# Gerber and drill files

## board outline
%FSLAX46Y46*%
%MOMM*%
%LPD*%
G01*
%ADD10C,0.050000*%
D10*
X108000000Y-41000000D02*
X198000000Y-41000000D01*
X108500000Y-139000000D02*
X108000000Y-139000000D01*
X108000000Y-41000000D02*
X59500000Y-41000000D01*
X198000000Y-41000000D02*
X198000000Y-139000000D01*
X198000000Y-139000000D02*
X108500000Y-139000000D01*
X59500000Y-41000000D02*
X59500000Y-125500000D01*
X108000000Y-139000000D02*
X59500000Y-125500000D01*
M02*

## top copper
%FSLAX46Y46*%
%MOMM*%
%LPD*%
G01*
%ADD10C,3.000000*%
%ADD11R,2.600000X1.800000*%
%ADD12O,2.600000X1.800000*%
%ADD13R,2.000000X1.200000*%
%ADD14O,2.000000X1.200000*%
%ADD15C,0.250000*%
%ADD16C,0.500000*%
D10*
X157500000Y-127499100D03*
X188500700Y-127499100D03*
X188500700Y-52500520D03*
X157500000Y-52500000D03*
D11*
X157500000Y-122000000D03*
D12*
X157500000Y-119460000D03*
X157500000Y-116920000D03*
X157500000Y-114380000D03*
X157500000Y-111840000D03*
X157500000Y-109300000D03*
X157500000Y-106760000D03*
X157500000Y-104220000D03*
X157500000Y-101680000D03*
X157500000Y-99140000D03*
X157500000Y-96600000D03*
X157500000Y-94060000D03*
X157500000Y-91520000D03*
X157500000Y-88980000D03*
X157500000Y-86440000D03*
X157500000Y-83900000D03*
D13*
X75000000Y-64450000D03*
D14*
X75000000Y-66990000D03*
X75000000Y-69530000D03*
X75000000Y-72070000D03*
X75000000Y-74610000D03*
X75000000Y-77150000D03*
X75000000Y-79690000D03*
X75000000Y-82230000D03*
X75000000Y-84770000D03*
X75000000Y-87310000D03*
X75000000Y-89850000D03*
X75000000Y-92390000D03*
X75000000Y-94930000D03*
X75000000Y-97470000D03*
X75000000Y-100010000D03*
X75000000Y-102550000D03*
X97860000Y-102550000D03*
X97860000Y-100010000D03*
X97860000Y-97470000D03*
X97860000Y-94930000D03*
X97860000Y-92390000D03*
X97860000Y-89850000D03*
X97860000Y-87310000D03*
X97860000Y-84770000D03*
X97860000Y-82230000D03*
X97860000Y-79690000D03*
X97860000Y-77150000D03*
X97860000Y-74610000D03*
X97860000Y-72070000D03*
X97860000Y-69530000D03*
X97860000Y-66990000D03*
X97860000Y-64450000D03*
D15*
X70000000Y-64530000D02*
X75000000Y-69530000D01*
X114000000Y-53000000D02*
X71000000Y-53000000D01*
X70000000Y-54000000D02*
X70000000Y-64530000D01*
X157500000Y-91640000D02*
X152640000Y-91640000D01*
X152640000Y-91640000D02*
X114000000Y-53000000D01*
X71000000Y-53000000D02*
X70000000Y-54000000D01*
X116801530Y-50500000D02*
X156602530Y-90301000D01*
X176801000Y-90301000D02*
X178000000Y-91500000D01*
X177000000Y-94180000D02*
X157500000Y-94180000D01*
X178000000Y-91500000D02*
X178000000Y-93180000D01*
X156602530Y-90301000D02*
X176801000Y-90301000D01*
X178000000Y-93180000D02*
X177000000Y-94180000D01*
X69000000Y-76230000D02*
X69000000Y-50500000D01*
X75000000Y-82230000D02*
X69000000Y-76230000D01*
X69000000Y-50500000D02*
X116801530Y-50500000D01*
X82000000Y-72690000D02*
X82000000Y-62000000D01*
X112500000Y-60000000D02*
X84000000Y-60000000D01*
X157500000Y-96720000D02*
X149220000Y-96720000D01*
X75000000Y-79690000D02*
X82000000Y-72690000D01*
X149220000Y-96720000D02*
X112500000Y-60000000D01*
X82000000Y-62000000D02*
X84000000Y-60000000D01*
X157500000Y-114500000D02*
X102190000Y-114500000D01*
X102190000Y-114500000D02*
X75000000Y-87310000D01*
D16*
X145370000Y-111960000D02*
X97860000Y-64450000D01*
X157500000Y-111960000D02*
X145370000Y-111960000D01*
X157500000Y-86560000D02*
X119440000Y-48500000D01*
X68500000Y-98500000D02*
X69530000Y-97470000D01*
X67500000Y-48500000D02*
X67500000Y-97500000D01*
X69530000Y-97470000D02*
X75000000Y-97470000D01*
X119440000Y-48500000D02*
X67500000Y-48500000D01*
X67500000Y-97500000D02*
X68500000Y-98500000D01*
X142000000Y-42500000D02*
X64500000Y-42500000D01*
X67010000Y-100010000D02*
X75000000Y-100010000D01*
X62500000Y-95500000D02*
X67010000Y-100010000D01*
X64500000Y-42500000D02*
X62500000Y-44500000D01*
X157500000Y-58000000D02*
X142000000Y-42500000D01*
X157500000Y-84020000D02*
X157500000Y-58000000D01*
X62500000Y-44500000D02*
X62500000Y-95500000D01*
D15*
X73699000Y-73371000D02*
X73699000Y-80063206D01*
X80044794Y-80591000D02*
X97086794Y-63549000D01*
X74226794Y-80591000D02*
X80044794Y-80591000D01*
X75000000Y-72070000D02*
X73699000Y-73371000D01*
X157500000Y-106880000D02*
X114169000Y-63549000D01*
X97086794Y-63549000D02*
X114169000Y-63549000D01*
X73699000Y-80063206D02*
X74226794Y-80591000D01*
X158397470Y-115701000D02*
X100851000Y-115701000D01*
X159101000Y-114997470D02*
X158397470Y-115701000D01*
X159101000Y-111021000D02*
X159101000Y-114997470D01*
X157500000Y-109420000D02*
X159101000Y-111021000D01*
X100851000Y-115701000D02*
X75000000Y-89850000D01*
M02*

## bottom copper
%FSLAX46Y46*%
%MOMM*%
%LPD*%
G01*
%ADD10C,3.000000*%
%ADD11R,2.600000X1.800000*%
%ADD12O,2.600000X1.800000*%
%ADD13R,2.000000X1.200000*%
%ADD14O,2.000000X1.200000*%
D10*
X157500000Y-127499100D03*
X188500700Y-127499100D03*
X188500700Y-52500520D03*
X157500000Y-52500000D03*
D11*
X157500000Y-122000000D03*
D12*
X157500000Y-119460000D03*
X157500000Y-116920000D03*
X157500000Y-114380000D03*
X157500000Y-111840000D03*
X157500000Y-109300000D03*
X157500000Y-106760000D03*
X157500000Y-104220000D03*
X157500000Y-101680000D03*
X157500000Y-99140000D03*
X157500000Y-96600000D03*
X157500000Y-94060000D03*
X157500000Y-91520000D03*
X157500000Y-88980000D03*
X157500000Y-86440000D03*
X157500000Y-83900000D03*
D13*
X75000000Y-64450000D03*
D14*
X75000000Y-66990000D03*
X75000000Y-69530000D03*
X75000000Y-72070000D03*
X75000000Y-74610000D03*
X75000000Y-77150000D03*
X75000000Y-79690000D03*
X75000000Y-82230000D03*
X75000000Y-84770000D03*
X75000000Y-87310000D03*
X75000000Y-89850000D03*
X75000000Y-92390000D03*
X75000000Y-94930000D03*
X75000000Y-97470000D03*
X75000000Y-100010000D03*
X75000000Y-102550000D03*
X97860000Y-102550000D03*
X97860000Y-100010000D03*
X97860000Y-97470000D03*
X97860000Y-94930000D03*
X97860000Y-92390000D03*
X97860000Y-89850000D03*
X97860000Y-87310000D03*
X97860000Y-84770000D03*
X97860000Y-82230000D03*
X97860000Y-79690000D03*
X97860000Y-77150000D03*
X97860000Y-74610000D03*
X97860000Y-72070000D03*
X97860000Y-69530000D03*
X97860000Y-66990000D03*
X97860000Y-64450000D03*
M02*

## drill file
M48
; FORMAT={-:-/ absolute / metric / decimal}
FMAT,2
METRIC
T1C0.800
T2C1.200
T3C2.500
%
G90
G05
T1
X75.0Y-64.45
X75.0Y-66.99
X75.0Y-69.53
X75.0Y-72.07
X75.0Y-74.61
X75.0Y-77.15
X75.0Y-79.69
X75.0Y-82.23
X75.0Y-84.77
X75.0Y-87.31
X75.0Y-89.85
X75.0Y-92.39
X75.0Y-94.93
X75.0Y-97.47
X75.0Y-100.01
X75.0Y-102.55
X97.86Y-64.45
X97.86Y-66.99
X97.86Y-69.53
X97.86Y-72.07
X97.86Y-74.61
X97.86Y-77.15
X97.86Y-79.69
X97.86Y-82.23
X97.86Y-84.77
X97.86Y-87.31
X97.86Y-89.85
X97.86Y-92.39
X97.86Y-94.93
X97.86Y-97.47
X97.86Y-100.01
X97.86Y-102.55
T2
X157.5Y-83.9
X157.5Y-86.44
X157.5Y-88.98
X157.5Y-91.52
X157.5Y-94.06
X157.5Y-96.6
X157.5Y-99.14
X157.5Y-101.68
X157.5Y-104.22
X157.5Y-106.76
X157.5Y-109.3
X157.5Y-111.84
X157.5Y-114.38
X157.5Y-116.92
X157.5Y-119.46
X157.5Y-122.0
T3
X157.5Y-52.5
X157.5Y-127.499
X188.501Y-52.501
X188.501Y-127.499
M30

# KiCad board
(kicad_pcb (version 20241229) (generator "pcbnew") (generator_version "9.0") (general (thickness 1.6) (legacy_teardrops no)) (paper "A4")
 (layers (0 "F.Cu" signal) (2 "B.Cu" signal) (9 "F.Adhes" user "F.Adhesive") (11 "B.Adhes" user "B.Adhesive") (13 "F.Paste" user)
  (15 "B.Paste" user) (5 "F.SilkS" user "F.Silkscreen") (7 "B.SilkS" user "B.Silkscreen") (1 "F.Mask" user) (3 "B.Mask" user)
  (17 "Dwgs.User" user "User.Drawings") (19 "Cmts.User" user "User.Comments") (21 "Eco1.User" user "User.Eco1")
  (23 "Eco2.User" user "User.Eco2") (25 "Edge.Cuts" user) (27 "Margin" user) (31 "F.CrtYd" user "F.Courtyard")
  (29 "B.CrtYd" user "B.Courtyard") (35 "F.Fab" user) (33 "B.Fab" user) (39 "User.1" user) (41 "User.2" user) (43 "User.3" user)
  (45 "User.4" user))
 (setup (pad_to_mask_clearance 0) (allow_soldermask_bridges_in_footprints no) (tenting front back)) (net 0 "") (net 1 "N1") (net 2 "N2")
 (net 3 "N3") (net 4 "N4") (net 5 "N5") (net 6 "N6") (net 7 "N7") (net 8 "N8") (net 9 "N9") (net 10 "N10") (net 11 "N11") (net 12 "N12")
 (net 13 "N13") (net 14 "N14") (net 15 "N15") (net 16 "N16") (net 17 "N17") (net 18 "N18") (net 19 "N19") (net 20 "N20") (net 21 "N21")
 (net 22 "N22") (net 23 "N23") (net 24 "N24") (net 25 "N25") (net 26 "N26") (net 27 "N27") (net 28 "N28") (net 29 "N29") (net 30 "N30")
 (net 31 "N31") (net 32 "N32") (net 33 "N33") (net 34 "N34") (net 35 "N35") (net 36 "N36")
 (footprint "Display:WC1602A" (layer "F.Cu") (at 157.5 122 90)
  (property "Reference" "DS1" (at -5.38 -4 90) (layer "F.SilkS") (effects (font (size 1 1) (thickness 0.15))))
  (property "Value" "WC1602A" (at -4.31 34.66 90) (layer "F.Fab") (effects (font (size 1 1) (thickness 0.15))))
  (pad "" thru_hole circle (at -5.4991 0 90) (size 3 3) (drill 2.5) (layers "*.Cu" "*.Mask") (remove_unused_layers no))
  (pad "" thru_hole circle (at -5.4991 31.0007 90) (size 3 3) (drill 2.5) (layers "*.Cu" "*.Mask") (remove_unused_layers no))
  (pad "" thru_hole circle (at 69.49948 31.0007 90) (size 3 3) (drill 2.5) (layers "*.Cu" "*.Mask") (remove_unused_layers no))
  (pad "" thru_hole circle (at 69.5 0 90) (size 3 3) (drill 2.5) (layers "*.Cu" "*.Mask") (remove_unused_layers no))
  (pad "1" thru_hole rect (at 0 0 90) (size 1.8 2.6) (drill 1.2) (layers "*.Cu" "*.Mask") (remove_unused_layers no) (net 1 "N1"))
  (pad "2" thru_hole oval (at 2.54 0 90) (size 1.8 2.6) (drill 1.2) (layers "*.Cu" "*.Mask") (remove_unused_layers no) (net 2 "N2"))
  (pad "3" thru_hole oval (at 5.08 0 90) (size 1.8 2.6) (drill 1.2) (layers "*.Cu" "*.Mask") (remove_unused_layers no) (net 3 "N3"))
  (pad "4" thru_hole oval (at 7.62 0 90) (size 1.8 2.6) (drill 1.2) (layers "*.Cu" "*.Mask") (remove_unused_layers no) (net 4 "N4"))
  (pad "5" thru_hole oval (at 10.16 0 90) (size 1.8 2.6) (drill 1.2) (layers "*.Cu" "*.Mask") (remove_unused_layers no) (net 1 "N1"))
  (pad "6" thru_hole oval (at 12.7 0 90) (size 1.8 2.6) (drill 1.2) (layers "*.Cu" "*.Mask") (remove_unused_layers no) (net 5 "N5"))
  (pad "7" thru_hole oval (at 15.24 0 90) (size 1.8 2.6) (drill 1.2) (layers "*.Cu" "*.Mask") (remove_unused_layers no) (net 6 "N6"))
  (pad "8" thru_hole oval (at 17.78 0 90) (size 1.8 2.6) (drill 1.2) (layers "*.Cu" "*.Mask") (remove_unused_layers no) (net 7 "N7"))
  (pad "9" thru_hole oval (at 20.32 0 90) (size 1.8 2.6) (drill 1.2) (layers "*.Cu" "*.Mask") (remove_unused_layers no) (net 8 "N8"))
  (pad "10" thru_hole oval (at 22.86 0 90) (size 1.8 2.6) (drill 1.2) (layers "*.Cu" "*.Mask") (remove_unused_layers no) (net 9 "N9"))
  (pad "11" thru_hole oval (at 25.4 0 90) (size 1.8 2.6) (drill 1.2) (layers "*.Cu" "*.Mask") (remove_unused_layers no) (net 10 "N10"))
  (pad "12" thru_hole oval (at 27.94 0 90) (size 1.8 2.6) (drill 1.2) (layers "*.Cu" "*.Mask") (remove_unused_layers no) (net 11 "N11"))
  (pad "13" thru_hole oval (at 30.48 0 90) (size 1.8 2.6) (drill 1.2) (layers "*.Cu" "*.Mask") (remove_unused_layers no) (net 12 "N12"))
  (pad "14" thru_hole oval (at 33.02 0 90) (size 1.8 2.6) (drill 1.2) (layers "*.Cu" "*.Mask") (remove_unused_layers no) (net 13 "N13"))
  (pad "15" thru_hole oval (at 35.56 0 90) (size 1.8 2.6) (drill 1.2) (layers "*.Cu" "*.Mask") (remove_unused_layers no) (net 2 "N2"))
  (pad "16" thru_hole oval (at 38.1 0 90) (size 1.8 2.6) (drill 1.2) (layers "*.Cu" "*.Mask") (remove_unused_layers no) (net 3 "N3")))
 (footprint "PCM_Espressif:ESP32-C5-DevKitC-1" (layer "F.Cu") (at 74.96012 64.45468)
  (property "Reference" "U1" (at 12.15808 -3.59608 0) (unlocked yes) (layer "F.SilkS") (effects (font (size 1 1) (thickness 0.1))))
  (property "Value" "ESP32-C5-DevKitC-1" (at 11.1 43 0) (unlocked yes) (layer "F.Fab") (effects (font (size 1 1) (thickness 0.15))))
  (pad "1" thru_hole rect (at 0.03988 -0.00468 270) (size 1.2 2) (drill 0.8) (layers "*.Cu" "*.Mask") (remove_unused_layers no)
   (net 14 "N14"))
  (pad "2" thru_hole oval (at 0.03988 2.53532 270) (size 1.2 2) (drill 0.8) (layers "*.Cu" "*.Mask") (remove_unused_layers no)
   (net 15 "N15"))
  (pad "3" thru_hole oval (at 0.03988 5.07532 270) (size 1.2 2) (drill 0.8) (layers "*.Cu" "*.Mask") (remove_unused_layers no)
   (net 12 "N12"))
  (pad "4" thru_hole oval (at 0.03988 7.61532 270) (size 1.2 2) (drill 0.8) (layers "*.Cu" "*.Mask") (remove_unused_layers no) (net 6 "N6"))
  (pad "5" thru_hole oval (at 0.03988 10.15532 270) (size 1.2 2) (drill 0.8) (layers "*.Cu" "*.Mask") (remove_unused_layers no)
   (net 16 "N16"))
  (pad "6" thru_hole oval (at 0.03988 12.69532 270) (size 1.2 2) (drill 0.8) (layers "*.Cu" "*.Mask") (remove_unused_layers no)
   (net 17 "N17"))
  (pad "7" thru_hole oval (at 0.03988 15.23532 270) (size 1.2 2) (drill 0.8) (layers "*.Cu" "*.Mask") (remove_unused_layers no)
   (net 10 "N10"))
  (pad "8" thru_hole oval (at 0.03988 17.77532 270) (size 1.2 2) (drill 0.8) (layers "*.Cu" "*.Mask") (remove_unused_layers no)
   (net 11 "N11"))
  (pad "9" thru_hole oval (at 0.03988 20.31532 270) (size 1.2 2) (drill 0.8) (layers "*.Cu" "*.Mask") (remove_unused_layers no)
   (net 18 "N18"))
  (pad "10" thru_hole oval (at 0.03988 22.85532 270) (size 1.2 2) (drill 0.8) (layers "*.Cu" "*.Mask") (remove_unused_layers no)
   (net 4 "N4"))
  (pad "11" thru_hole oval (at 0.03988 25.39532 270) (size 1.2 2) (drill 0.8) (layers "*.Cu" "*.Mask") (remove_unused_layers no)
   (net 5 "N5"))
  (pad "12" thru_hole oval (at 0.03988 27.93532 270) (size 1.2 2) (drill 0.8) (layers "*.Cu" "*.Mask") (remove_unused_layers no)
   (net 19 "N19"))
  (pad "13" thru_hole oval (at 0.03988 30.47532 270) (size 1.2 2) (drill 0.8) (layers "*.Cu" "*.Mask") (remove_unused_layers no)
   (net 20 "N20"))
  (pad "14" thru_hole oval (at 0.03988 33.01532 270) (size 1.2 2) (drill 0.8) (layers "*.Cu" "*.Mask") (remove_unused_layers no)
   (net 2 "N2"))
  (pad "15" thru_hole oval (at 0.03988 35.55532 270) (size 1.2 2) (drill 0.8) (layers "*.Cu" "*.Mask") (remove_unused_layers no)
   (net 3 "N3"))
  (pad "16" thru_hole oval (at 0.03988 38.09532 270) (size 1.2 2) (drill 0.8) (layers "*.Cu" "*.Mask") (remove_unused_layers no)
   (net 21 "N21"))
  (pad "17" thru_hole oval (at 22.89988 38.09532 270) (size 1.2 2) (drill 0.8) (layers "*.Cu" "*.Mask") (remove_unused_layers no)
   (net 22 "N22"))
  (pad "18" thru_hole oval (at 22.89988 35.55532 270) (size 1.2 2) (drill 0.8) (layers "*.Cu" "*.Mask") (remove_unused_layers no)
   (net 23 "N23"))
  (pad "19" thru_hole oval (at 22.89988 33.01532 270) (size 1.2 2) (drill 0.8) (layers "*.Cu" "*.Mask") (remove_unused_layers no)
   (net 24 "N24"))
  (pad "20" thru_hole oval (at 22.89988 30.47532 270) (size 1.2 2) (drill 0.8) (layers "*.Cu" "*.Mask") (remove_unused_layers no)
   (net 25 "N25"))
  (pad "21" thru_hole oval (at 22.89988 27.93532 270) (size 1.2 2) (drill 0.8) (layers "*.Cu" "*.Mask") (remove_unused_layers no)
   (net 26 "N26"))
  (pad "22" thru_hole oval (at 22.89988 25.39532 270) (size 1.2 2) (drill 0.8) (layers "*.Cu" "*.Mask") (remove_unused_layers no)
   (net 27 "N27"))
  (pad "23" thru_hole oval (at 22.89988 22.85532 270) (size 1.2 2) (drill 0.8) (layers "*.Cu" "*.Mask") (remove_unused_layers no)
   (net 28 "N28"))
  (pad "24" thru_hole oval (at 22.89988 20.31532 270) (size 1.2 2) (drill 0.8) (layers "*.Cu" "*.Mask") (remove_unused_layers no)
   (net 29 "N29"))
  (pad "25" thru_hole oval (at 22.89988 17.77532 270) (size 1.2 2) (drill 0.8) (layers "*.Cu" "*.Mask") (remove_unused_layers no)
   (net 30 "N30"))
  (pad "26" thru_hole oval (at 22.89988 15.23532 270) (size 1.2 2) (drill 0.8) (layers "*.Cu" "*.Mask") (remove_unused_layers no)
   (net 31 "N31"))
  (pad "27" thru_hole oval (at 22.89988 12.69532 270) (size 1.2 2) (drill 0.8) (layers "*.Cu" "*.Mask") (remove_unused_layers no)
   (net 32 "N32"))
  (pad "28" thru_hole oval (at 22.89988 10.15532 270) (size 1.2 2) (drill 0.8) (layers "*.Cu" "*.Mask") (remove_unused_layers no)
   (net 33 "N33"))
  (pad "29" thru_hole oval (at 22.89988 7.61532 270) (size 1.2 2) (drill 0.8) (layers "*.Cu" "*.Mask") (remove_unused_layers no)
   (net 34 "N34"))
  (pad "30" thru_hole oval (at 22.89988 5.07532 270) (size 1.2 2) (drill 0.8) (layers "*.Cu" "*.Mask") (remove_unused_layers no)
   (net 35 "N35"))
  (pad "31" thru_hole oval (at 22.89988 2.53532 270) (size 1.2 2) (drill 0.8) (layers "*.Cu" "*.Mask") (remove_unused_layers no)
   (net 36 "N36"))
  (pad "32" thru_hole oval (at 22.89988 -0.00468 270) (size 1.2 2) (drill 0.8) (layers "*.Cu" "*.Mask") (remove_unused_layers no)
   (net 1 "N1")))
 (gr_line (start 108 41) (end 198 41) (stroke (width 0.05) (type default)) (layer "Edge.Cuts"))
 (gr_line (start 108.5 139) (end 108 139) (stroke (width 0.05) (type default)) (layer "Edge.Cuts"))
 (gr_line (start 108 41) (end 59.5 41) (stroke (width 0.05) (type default)) (layer "Edge.Cuts"))
 (gr_line (start 198 41) (end 198 139) (stroke (width 0.05) (type default)) (layer "Edge.Cuts"))
 (gr_line (start 198 139) (end 108.5 139) (stroke (width 0.05) (type default)) (layer "Edge.Cuts"))
 (gr_line (start 59.5 41) (end 59.5 125.5) (stroke (width 0.05) (type default)) (layer "Edge.Cuts"))
 (gr_line (start 108 139) (end 59.5 125.5) (stroke (width 0.05) (type default)) (layer "Edge.Cuts"))
 (segment (start 70 64.53) (end 75 69.53) (width 0.25) (layer "F.Cu") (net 12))
 (segment (start 114 53) (end 71 53) (width 0.25) (layer "F.Cu") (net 12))
 (segment (start 70 54) (end 70 64.53) (width 0.25) (layer "F.Cu") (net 12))
 (segment (start 157.5 91.64) (end 152.64 91.64) (width 0.25) (layer "F.Cu") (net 12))
 (segment (start 152.64 91.64) (end 114 53) (width 0.25) (layer "F.Cu") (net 12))
 (segment (start 71 53) (end 70 54) (width 0.25) (layer "F.Cu") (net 12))
 (segment (start 116.80153 50.5) (end 156.60253 90.301) (width 0.25) (layer "F.Cu") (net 11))
 (segment (start 176.801 90.301) (end 178 91.5) (width 0.25) (layer "F.Cu") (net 11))
 (segment (start 177 94.18) (end 157.5 94.18) (width 0.25) (layer "F.Cu") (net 11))
 (segment (start 178 91.5) (end 178 93.18) (width 0.25) (layer "F.Cu") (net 11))
 (segment (start 156.60253 90.301) (end 176.801 90.301) (width 0.25) (layer "F.Cu") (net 11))
 (segment (start 178 93.18) (end 177 94.18) (width 0.25) (layer "F.Cu") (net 11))
 (segment (start 69 76.23) (end 69 50.5) (width 0.25) (layer "F.Cu") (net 11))
 (segment (start 75 82.23) (end 69 76.23) (width 0.25) (layer "F.Cu") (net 11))
 (segment (start 69 50.5) (end 116.80153 50.5) (width 0.25) (layer "F.Cu") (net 11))
 (segment (start 82 72.69) (end 82 62) (width 0.25) (layer "F.Cu") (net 10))
 (segment (start 112.5 60) (end 84 60) (width 0.25) (layer "F.Cu") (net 10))
 (segment (start 157.5 96.72) (end 149.22 96.72) (width 0.25) (layer "F.Cu") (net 10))
 (segment (start 75 79.69) (end 82 72.69) (width 0.25) (layer "F.Cu") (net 10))
 (segment (start 149.22 96.72) (end 112.5 60) (width 0.25) (layer "F.Cu") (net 10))
 (segment (start 82 62) (end 84 60) (width 0.25) (layer "F.Cu") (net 10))
 (segment (start 157.5 114.5) (end 102.19 114.5) (width 0.25) (layer "F.Cu") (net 4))
 (segment (start 102.19 114.5) (end 75 87.31) (width 0.25) (layer "F.Cu") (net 4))
 (segment (start 145.37 111.96) (end 97.86 64.45) (width 0.5) (layer "F.Cu") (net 1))
 (segment (start 157.5 111.96) (end 145.37 111.96) (width 0.5) (layer "F.Cu") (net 1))
 (segment (start 157.5 86.56) (end 119.44 48.5) (width 0.5) (layer "F.Cu") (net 2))
 (segment (start 68.5 98.5) (end 69.53 97.47) (width 0.5) (layer "F.Cu") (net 2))
 (segment (start 67.5 48.5) (end 67.5 97.5) (width 0.5) (layer "F.Cu") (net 2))
 (segment (start 69.53 97.47) (end 75 97.47) (width 0.5) (layer "F.Cu") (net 2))
 (segment (start 119.44 48.5) (end 67.5 48.5) (width 0.5) (layer "F.Cu") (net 2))
 (segment (start 67.5 97.5) (end 68.5 98.5) (width 0.5) (layer "F.Cu") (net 2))
 (segment (start 142 42.5) (end 64.5 42.5) (width 0.5) (layer "F.Cu") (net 3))
 (segment (start 67.01 100.01) (end 75 100.01) (width 0.5) (layer "F.Cu") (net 3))
 (segment (start 62.5 95.5) (end 67.01 100.01) (width 0.5) (layer "F.Cu") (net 3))
 (segment (start 64.5 42.5) (end 62.5 44.5) (width 0.5) (layer "F.Cu") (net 3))
 (segment (start 157.5 58) (end 142 42.5) (width 0.5) (layer "F.Cu") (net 3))
 (segment (start 157.5 84.02) (end 157.5 58) (width 0.5) (layer "F.Cu") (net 3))
 (segment (start 62.5 44.5) (end 62.5 95.5) (width 0.5) (layer "F.Cu") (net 3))
 (segment (start 73.699 73.371) (end 73.699 80.063206) (width 0.25) (layer "F.Cu") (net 6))
 (segment (start 80.044794 80.591) (end 97.086794 63.549) (width 0.25) (layer "F.Cu") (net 6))
 (segment (start 74.226794 80.591) (end 80.044794 80.591) (width 0.25) (layer "F.Cu") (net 6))
 (segment (start 75 72.07) (end 73.699 73.371) (width 0.25) (layer "F.Cu") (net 6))
 (segment (start 157.5 106.88) (end 114.169 63.549) (width 0.25) (layer "F.Cu") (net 6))
 (segment (start 97.086794 63.549) (end 114.169 63.549) (width 0.25) (layer "F.Cu") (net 6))
 (segment (start 73.699 80.063206) (end 74.226794 80.591) (width 0.25) (layer "F.Cu") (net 6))
 (segment (start 158.39747 115.701) (end 100.851 115.701) (width 0.25) (layer "F.Cu") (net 5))
 (segment (start 159.101 114.99747) (end 158.39747 115.701) (width 0.25) (layer "F.Cu") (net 5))
 (segment (start 159.101 111.021) (end 159.101 114.99747) (width 0.25) (layer "F.Cu") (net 5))
 (segment (start 157.5 109.42) (end 159.101 111.021) (width 0.25) (layer "F.Cu") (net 5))
 (segment (start 100.851 115.701) (end 75 89.85) (width 0.25) (layer "F.Cu") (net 5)))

